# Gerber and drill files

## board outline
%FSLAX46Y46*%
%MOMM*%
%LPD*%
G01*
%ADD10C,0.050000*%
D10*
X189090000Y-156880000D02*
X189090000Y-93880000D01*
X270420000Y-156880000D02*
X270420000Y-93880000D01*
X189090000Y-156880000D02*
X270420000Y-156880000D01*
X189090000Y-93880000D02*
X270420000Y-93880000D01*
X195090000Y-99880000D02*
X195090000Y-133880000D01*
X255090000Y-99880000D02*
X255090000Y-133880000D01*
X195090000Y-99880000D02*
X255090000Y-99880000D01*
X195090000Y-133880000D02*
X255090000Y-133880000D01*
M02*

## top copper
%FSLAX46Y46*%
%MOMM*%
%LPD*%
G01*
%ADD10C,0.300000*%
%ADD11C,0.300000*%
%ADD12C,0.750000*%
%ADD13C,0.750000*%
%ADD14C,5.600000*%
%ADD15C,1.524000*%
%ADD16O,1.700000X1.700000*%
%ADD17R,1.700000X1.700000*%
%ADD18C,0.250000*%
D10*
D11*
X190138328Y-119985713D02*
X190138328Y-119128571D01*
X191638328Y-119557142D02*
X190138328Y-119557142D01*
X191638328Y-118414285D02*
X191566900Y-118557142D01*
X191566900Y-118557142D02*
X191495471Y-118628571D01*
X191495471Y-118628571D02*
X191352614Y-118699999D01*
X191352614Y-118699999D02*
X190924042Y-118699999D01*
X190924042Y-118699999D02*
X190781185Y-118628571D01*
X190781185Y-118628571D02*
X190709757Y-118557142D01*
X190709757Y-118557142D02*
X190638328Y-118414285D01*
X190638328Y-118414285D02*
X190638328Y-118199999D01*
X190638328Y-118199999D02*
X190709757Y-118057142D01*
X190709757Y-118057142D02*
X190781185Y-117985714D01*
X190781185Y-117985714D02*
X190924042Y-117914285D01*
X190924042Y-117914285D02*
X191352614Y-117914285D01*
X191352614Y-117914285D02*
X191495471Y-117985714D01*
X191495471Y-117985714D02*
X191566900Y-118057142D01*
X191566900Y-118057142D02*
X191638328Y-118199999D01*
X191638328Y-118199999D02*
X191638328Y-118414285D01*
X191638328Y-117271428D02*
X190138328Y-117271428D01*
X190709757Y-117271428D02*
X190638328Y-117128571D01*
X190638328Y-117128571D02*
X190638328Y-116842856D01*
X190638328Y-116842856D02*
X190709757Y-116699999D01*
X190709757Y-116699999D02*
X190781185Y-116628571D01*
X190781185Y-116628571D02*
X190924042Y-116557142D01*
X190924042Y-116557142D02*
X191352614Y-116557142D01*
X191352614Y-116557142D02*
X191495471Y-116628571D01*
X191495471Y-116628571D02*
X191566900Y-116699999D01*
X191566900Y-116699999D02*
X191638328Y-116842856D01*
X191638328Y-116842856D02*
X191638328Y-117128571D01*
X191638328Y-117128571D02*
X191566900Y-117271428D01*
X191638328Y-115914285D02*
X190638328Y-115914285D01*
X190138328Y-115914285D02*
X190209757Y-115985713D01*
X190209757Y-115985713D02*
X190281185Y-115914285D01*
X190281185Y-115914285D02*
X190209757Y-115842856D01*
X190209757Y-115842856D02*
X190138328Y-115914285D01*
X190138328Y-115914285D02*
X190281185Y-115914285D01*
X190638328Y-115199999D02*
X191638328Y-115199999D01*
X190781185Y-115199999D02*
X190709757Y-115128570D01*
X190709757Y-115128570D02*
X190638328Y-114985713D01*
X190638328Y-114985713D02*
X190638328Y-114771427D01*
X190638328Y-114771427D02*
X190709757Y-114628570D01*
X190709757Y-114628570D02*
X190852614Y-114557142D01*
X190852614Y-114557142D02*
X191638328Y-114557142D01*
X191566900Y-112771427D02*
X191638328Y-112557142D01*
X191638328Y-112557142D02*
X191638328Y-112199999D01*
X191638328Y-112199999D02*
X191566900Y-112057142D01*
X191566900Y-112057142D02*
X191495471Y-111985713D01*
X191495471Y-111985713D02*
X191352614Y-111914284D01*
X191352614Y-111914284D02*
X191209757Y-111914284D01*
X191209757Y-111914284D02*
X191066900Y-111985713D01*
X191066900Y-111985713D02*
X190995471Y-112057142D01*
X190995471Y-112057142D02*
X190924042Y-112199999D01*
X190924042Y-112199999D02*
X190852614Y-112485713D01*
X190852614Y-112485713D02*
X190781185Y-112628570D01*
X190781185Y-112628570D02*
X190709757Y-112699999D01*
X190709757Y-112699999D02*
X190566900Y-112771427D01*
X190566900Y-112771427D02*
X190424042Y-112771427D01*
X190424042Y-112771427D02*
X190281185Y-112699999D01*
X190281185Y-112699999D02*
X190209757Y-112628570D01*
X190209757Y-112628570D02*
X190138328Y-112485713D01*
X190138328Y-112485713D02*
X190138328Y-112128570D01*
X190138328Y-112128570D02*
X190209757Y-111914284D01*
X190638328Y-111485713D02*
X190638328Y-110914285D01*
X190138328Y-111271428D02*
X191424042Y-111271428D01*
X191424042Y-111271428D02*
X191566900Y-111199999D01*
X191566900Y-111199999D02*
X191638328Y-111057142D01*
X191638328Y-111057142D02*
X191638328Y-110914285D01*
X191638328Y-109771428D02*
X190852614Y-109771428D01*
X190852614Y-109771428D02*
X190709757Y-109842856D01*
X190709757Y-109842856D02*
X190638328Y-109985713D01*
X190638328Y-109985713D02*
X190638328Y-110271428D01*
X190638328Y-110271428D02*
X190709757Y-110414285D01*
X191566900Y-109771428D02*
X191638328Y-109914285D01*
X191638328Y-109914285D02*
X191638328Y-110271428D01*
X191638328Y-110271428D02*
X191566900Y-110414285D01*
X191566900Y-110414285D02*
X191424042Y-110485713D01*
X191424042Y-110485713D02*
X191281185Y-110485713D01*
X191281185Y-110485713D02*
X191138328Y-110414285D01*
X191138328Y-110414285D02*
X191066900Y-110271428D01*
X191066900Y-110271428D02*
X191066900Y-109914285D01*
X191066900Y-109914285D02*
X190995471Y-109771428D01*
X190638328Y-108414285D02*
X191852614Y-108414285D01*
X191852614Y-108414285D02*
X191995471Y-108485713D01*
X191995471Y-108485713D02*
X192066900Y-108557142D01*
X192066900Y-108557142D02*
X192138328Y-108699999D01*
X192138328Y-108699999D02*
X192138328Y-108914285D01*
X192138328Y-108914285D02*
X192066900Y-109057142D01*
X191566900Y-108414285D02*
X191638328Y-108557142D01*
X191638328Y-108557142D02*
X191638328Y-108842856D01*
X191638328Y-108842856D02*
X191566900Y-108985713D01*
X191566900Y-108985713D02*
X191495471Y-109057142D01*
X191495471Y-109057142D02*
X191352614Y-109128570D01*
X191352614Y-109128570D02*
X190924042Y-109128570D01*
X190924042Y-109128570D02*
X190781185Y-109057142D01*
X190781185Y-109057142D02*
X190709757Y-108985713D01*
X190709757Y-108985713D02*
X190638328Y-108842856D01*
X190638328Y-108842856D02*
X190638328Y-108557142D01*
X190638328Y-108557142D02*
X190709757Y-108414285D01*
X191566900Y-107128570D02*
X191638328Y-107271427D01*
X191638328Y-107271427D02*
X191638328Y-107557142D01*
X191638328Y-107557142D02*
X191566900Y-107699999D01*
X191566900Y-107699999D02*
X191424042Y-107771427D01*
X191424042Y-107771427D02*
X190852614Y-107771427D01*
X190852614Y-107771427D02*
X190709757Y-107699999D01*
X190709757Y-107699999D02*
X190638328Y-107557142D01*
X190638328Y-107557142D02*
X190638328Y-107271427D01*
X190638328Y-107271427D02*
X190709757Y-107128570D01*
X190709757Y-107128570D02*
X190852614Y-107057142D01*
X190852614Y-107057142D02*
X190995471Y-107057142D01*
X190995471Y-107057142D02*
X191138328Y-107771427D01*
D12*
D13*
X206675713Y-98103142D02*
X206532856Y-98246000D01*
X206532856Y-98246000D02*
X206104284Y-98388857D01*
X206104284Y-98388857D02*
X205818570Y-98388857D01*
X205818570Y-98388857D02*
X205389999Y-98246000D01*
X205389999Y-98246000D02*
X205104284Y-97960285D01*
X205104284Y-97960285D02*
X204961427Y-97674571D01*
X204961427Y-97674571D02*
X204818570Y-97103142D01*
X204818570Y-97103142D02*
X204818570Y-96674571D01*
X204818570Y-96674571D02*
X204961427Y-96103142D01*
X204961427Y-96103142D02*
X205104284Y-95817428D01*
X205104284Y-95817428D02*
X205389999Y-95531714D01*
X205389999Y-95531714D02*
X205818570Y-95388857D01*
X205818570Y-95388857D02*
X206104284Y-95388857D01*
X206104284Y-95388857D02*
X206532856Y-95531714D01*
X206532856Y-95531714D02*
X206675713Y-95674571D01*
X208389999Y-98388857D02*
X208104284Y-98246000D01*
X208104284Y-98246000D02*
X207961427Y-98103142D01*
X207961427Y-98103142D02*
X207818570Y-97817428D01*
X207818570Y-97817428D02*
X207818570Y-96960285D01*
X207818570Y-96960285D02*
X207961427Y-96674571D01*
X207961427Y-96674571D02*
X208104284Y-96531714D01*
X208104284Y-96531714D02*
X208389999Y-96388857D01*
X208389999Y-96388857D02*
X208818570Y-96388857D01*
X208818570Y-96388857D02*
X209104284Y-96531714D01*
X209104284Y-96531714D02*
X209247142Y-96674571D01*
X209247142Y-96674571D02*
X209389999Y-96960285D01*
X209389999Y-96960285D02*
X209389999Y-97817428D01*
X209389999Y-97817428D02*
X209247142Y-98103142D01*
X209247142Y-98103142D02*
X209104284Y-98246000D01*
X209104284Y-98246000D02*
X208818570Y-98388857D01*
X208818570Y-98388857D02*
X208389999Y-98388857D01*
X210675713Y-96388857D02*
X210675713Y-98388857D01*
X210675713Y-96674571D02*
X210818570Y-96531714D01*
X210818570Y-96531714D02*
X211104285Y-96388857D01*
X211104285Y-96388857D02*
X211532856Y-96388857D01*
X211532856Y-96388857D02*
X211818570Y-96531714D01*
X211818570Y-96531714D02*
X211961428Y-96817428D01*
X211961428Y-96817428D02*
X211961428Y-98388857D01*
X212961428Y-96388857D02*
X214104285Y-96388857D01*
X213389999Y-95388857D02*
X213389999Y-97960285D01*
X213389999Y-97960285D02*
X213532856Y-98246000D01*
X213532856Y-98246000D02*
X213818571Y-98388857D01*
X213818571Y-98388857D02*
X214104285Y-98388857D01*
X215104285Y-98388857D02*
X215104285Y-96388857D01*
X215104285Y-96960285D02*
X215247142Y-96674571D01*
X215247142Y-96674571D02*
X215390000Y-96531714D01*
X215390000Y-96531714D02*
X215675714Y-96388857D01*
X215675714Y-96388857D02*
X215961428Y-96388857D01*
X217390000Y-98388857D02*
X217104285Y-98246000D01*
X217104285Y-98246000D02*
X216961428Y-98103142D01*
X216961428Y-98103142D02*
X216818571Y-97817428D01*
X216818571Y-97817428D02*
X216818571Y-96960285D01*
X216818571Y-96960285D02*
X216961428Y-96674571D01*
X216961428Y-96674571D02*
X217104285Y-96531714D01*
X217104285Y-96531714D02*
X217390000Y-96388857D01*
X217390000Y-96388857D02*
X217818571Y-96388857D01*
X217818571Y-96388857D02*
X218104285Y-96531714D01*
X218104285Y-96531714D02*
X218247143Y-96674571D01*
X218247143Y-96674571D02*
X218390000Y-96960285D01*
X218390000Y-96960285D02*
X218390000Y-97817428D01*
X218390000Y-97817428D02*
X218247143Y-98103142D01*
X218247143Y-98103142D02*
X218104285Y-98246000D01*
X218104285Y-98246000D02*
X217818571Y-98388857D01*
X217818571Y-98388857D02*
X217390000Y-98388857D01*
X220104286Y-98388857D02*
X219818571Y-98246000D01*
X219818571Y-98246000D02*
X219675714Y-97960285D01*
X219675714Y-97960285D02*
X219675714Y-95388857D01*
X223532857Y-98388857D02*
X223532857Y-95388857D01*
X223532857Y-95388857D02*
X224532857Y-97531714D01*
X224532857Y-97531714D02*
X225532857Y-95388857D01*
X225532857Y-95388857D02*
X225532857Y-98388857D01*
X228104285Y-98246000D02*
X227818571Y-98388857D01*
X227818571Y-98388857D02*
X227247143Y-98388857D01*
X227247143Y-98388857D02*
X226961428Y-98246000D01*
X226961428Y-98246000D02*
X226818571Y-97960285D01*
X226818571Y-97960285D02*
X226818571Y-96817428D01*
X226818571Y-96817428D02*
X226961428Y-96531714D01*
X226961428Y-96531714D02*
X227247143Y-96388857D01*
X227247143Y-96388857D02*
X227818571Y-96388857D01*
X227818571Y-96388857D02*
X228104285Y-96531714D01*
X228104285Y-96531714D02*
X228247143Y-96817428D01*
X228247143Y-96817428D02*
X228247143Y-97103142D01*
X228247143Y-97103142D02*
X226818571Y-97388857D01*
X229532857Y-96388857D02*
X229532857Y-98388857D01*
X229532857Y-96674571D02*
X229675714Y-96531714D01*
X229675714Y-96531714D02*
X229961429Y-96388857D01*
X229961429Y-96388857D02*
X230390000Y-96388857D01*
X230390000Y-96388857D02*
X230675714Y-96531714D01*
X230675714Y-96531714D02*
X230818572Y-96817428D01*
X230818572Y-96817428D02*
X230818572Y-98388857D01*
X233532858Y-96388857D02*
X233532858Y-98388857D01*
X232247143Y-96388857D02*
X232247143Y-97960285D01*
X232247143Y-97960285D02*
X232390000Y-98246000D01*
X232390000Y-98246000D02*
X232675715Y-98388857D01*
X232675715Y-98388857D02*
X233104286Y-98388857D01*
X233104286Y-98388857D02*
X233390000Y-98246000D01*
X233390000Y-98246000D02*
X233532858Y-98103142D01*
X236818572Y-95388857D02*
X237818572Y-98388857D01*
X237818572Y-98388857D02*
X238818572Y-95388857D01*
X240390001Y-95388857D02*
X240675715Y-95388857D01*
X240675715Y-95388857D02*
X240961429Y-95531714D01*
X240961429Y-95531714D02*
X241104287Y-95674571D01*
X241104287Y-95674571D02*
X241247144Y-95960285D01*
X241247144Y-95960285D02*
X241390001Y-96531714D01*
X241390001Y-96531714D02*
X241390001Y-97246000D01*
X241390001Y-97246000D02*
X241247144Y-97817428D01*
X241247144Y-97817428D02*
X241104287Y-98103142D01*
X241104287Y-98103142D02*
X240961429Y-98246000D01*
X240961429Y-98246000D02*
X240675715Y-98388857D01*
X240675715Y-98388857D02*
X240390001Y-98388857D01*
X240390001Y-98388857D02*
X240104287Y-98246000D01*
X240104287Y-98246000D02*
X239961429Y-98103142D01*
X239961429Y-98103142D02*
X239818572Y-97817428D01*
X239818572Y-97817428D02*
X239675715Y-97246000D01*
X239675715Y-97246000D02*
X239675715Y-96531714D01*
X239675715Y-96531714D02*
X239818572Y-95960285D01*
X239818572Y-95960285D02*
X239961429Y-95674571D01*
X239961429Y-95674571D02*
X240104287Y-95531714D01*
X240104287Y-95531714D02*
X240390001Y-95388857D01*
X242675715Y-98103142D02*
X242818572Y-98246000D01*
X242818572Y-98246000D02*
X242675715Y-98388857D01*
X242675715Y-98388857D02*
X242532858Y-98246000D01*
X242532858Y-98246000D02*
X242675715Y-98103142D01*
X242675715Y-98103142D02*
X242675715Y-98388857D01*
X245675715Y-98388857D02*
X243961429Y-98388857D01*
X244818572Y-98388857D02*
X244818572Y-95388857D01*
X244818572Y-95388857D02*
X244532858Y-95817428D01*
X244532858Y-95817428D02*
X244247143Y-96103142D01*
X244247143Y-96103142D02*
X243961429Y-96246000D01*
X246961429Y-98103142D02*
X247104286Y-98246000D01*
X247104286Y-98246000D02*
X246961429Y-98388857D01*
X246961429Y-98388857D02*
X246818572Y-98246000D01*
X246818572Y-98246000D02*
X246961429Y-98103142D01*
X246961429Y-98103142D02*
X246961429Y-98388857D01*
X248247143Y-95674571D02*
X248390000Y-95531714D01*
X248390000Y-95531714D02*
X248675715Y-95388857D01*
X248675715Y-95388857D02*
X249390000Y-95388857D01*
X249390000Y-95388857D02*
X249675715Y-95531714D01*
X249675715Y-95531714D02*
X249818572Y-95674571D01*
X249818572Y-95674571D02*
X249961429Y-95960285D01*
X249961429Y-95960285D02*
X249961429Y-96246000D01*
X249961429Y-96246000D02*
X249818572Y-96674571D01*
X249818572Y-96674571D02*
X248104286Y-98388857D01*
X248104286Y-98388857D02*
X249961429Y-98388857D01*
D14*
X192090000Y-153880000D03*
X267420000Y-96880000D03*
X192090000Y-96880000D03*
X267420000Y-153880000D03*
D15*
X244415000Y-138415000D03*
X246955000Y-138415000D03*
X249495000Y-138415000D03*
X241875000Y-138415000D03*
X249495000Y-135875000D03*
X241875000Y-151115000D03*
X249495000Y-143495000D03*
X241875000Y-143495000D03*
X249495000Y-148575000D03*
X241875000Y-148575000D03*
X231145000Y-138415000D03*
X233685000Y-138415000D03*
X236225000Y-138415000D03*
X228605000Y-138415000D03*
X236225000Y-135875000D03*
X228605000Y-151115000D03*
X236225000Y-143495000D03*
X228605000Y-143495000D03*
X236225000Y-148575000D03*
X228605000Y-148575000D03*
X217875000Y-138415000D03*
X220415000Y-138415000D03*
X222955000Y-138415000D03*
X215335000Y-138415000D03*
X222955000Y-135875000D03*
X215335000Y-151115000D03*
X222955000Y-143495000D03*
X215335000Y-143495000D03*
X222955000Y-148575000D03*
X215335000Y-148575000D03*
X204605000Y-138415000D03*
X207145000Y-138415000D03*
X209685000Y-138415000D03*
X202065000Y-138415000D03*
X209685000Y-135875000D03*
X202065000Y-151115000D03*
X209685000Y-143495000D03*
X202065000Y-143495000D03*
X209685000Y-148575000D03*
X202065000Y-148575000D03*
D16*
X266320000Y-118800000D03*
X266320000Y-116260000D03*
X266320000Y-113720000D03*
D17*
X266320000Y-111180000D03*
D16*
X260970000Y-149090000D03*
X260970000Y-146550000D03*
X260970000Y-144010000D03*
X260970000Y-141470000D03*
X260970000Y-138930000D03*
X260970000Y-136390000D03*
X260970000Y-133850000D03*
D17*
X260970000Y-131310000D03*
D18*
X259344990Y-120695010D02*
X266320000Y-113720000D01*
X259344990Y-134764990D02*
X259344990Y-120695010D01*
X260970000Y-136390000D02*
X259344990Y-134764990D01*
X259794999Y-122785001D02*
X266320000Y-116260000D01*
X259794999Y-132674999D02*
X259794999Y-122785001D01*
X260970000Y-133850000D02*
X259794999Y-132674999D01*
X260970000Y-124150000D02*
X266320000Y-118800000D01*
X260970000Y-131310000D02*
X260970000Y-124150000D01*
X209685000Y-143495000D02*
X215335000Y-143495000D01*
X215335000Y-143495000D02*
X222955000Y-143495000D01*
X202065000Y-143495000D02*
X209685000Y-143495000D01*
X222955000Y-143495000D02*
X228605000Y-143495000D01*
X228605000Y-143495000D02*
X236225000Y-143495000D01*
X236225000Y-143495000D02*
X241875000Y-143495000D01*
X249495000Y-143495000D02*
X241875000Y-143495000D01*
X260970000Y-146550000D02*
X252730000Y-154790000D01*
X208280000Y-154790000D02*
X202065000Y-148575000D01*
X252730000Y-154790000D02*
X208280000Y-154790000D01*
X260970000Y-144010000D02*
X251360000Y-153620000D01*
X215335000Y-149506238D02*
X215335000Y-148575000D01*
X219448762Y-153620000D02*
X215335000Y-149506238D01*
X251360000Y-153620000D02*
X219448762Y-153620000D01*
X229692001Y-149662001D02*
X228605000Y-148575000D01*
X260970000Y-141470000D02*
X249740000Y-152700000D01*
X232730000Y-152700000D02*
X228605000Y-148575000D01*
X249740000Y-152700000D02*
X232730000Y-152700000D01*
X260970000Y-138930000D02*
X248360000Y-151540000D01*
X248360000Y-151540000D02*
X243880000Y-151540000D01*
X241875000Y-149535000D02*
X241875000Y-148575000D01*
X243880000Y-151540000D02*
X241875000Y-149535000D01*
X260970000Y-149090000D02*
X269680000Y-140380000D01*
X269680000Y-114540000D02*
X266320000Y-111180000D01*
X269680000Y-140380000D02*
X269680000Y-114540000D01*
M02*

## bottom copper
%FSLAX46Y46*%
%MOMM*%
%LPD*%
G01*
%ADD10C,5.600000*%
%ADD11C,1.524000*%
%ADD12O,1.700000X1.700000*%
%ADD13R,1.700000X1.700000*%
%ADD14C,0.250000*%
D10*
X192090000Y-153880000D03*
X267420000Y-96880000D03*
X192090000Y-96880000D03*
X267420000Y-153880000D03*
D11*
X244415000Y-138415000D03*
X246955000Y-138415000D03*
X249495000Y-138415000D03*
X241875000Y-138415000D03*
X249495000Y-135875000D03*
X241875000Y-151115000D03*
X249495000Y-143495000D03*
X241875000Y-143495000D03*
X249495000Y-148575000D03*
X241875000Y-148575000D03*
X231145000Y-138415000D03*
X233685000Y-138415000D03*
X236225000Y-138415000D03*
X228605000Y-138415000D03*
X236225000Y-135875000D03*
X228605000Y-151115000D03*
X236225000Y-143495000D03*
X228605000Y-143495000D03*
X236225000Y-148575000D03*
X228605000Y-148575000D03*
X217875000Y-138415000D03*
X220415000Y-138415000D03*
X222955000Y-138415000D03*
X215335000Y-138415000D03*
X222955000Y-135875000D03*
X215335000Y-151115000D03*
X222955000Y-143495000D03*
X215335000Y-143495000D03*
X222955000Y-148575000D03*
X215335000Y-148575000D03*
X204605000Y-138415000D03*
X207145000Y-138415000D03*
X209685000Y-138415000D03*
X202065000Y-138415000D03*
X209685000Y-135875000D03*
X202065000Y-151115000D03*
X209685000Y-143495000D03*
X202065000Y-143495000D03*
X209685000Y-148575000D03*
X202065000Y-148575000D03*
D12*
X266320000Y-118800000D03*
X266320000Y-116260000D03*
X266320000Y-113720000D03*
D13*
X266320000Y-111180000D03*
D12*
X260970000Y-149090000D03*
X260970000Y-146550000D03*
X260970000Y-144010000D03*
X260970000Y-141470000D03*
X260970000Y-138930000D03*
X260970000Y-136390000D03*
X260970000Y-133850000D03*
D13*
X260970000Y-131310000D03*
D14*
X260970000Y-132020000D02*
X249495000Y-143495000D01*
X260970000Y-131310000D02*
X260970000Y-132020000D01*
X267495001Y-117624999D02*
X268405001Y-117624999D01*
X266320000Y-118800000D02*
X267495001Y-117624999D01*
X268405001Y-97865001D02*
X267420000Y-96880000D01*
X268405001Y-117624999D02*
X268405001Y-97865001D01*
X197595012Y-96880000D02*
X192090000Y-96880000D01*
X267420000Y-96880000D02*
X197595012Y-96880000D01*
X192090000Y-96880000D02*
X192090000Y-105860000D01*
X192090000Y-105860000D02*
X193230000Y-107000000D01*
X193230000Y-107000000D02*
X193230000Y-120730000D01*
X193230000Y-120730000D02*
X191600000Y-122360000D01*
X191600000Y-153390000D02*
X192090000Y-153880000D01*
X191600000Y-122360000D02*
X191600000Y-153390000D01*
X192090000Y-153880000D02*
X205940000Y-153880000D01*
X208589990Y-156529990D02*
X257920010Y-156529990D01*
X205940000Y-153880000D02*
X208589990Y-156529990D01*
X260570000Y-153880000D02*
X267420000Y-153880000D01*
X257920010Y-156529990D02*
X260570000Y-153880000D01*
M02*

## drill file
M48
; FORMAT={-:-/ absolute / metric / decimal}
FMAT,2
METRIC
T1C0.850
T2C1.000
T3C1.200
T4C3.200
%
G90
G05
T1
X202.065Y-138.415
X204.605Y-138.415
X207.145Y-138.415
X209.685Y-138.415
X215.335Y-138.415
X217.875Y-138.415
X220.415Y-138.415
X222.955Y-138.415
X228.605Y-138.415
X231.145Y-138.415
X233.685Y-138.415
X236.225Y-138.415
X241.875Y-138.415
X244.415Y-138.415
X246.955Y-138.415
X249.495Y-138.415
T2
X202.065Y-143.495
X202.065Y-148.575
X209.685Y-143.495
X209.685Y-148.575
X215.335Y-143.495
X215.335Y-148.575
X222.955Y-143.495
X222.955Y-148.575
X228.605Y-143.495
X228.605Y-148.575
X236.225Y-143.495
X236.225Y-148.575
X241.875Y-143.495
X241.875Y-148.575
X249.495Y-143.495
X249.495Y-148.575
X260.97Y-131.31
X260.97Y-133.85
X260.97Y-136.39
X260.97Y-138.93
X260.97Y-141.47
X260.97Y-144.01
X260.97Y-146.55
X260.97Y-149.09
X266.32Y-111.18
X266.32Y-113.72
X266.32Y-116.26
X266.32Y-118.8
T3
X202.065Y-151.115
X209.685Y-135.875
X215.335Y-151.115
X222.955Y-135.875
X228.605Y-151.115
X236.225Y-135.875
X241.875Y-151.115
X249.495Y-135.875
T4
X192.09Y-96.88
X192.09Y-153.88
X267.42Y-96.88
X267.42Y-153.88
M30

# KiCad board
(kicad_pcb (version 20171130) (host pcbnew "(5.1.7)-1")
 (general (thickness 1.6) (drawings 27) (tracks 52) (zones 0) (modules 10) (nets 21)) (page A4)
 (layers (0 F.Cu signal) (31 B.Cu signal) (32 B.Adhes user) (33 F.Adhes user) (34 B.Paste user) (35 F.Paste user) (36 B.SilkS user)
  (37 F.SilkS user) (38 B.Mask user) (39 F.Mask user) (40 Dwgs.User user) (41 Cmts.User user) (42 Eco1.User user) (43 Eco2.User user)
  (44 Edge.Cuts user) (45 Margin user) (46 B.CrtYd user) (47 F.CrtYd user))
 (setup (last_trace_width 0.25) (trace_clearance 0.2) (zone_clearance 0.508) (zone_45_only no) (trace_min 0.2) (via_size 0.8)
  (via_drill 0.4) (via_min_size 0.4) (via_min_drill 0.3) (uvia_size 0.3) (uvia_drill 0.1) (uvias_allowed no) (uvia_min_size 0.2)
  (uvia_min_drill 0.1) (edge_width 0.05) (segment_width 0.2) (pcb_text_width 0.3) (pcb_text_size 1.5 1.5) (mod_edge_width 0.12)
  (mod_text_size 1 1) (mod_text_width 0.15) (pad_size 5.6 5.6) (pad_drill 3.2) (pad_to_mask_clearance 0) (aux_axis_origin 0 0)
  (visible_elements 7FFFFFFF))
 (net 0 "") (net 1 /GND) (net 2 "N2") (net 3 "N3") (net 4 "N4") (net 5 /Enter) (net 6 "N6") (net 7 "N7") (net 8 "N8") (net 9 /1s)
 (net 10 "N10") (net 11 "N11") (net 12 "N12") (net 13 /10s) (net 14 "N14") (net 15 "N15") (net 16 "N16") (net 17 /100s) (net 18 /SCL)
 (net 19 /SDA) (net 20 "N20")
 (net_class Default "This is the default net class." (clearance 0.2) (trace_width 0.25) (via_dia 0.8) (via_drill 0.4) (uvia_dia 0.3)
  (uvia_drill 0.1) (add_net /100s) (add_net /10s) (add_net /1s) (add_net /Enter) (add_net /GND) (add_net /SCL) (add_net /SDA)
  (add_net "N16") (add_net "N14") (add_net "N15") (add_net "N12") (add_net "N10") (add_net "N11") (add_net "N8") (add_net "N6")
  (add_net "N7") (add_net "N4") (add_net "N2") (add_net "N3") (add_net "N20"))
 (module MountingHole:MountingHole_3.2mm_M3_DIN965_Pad (layer F.Cu) (at 192.09 153.88)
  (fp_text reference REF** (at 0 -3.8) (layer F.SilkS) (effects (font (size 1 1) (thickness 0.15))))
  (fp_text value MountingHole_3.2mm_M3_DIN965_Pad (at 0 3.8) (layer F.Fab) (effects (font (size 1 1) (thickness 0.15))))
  (pad 1 thru_hole circle (at 0 0) (size 5.6 5.6) (drill 3.2) (layers *.Cu *.Mask) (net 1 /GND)))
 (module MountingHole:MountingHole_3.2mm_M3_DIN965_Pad (layer F.Cu) (at 267.42 96.88)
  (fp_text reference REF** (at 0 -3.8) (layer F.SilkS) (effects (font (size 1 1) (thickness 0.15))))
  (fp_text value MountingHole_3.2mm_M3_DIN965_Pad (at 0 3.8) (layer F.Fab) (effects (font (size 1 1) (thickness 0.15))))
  (pad 1 thru_hole circle (at 0 0) (size 5.6 5.6) (drill 3.2) (layers *.Cu *.Mask) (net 1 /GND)))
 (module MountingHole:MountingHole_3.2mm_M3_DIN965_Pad (layer F.Cu) (at 192.09 96.88)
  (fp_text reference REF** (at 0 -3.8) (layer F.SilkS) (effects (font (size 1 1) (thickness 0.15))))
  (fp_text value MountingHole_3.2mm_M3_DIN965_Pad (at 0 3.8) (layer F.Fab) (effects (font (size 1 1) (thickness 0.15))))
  (pad 1 thru_hole circle (at 0 0) (size 5.6 5.6) (drill 3.2) (layers *.Cu *.Mask) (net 1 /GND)))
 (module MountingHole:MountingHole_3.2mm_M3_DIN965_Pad (layer F.Cu) (at 267.42 153.88)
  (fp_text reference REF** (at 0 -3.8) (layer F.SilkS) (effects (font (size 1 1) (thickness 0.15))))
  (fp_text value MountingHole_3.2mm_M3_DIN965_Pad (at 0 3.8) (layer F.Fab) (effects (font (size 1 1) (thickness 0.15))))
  (pad 1 thru_hole circle (at 0 0) (size 5.6 5.6) (drill 3.2) (layers *.Cu *.Mask) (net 1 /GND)))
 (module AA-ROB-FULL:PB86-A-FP (layer F.Cu) (at 239.515 134.995)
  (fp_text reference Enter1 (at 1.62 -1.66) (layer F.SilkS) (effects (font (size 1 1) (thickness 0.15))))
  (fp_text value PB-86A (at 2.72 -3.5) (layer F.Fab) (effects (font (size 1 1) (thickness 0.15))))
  (pad 5 thru_hole circle (at 4.9 3.42) (size 1.524 1.524) (drill 0.85) (layers *.Cu *.Mask) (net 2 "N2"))
  (pad 6 thru_hole circle (at 7.44 3.42) (size 1.524 1.524) (drill 0.85) (layers *.Cu *.Mask) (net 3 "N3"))
  (pad 7 thru_hole circle (at 9.98 3.42) (size 1.524 1.524) (drill 0.85) (layers *.Cu *.Mask))
  (pad 4 thru_hole circle (at 2.36 3.42) (size 1.524 1.524) (drill 0.85) (layers *.Cu *.Mask))
  (pad 8 thru_hole circle (at 9.98 0.88) (size 1.524 1.524) (drill 1.2) (layers *.Cu *.Mask))
  (pad 8 thru_hole circle (at 2.36 16.12) (size 1.524 1.524) (drill 1.2) (layers *.Cu *.Mask))
  (pad 1 thru_hole circle (at 9.98 8.5) (size 1.524 1.524) (drill 1) (layers *.Cu *.Mask) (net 1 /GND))
  (pad 1 thru_hole circle (at 2.36 8.5) (size 1.524 1.524) (drill 1) (layers *.Cu *.Mask) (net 1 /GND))
  (pad 3 thru_hole circle (at 9.98 13.58) (size 1.524 1.524) (drill 1) (layers *.Cu *.Mask) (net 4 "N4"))
  (pad 2 thru_hole circle (at 2.36 13.58) (size 1.524 1.524) (drill 1) (layers *.Cu *.Mask) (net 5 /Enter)))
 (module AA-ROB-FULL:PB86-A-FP (layer F.Cu) (at 226.245 134.995)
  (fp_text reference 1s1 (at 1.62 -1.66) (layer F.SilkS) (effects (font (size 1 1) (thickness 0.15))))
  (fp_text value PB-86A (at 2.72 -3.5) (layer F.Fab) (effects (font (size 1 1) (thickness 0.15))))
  (pad 5 thru_hole circle (at 4.9 3.42) (size 1.524 1.524) (drill 0.85) (layers *.Cu *.Mask) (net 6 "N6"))
  (pad 6 thru_hole circle (at 7.44 3.42) (size 1.524 1.524) (drill 0.85) (layers *.Cu *.Mask) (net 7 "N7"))
  (pad 7 thru_hole circle (at 9.98 3.42) (size 1.524 1.524) (drill 0.85) (layers *.Cu *.Mask))
  (pad 4 thru_hole circle (at 2.36 3.42) (size 1.524 1.524) (drill 0.85) (layers *.Cu *.Mask))
  (pad 8 thru_hole circle (at 9.98 0.88) (size 1.524 1.524) (drill 1.2) (layers *.Cu *.Mask))
  (pad 8 thru_hole circle (at 2.36 16.12) (size 1.524 1.524) (drill 1.2) (layers *.Cu *.Mask))
  (pad 1 thru_hole circle (at 9.98 8.5) (size 1.524 1.524) (drill 1) (layers *.Cu *.Mask) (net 1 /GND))
  (pad 1 thru_hole circle (at 2.36 8.5) (size 1.524 1.524) (drill 1) (layers *.Cu *.Mask) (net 1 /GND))
  (pad 3 thru_hole circle (at 9.98 13.58) (size 1.524 1.524) (drill 1) (layers *.Cu *.Mask) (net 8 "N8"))
  (pad 2 thru_hole circle (at 2.36 13.58) (size 1.524 1.524) (drill 1) (layers *.Cu *.Mask) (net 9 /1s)))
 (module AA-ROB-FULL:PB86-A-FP (layer F.Cu) (at 212.975 134.995)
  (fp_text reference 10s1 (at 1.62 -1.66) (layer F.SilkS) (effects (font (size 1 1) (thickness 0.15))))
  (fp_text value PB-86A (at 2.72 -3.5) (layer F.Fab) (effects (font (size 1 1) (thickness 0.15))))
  (pad 5 thru_hole circle (at 4.9 3.42) (size 1.524 1.524) (drill 0.85) (layers *.Cu *.Mask) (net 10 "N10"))
  (pad 6 thru_hole circle (at 7.44 3.42) (size 1.524 1.524) (drill 0.85) (layers *.Cu *.Mask) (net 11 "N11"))
  (pad 7 thru_hole circle (at 9.98 3.42) (size 1.524 1.524) (drill 0.85) (layers *.Cu *.Mask))
  (pad 4 thru_hole circle (at 2.36 3.42) (size 1.524 1.524) (drill 0.85) (layers *.Cu *.Mask))
  (pad 8 thru_hole circle (at 9.98 0.88) (size 1.524 1.524) (drill 1.2) (layers *.Cu *.Mask))
  (pad 8 thru_hole circle (at 2.36 16.12) (size 1.524 1.524) (drill 1.2) (layers *.Cu *.Mask))
  (pad 1 thru_hole circle (at 9.98 8.5) (size 1.524 1.524) (drill 1) (layers *.Cu *.Mask) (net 1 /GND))
  (pad 1 thru_hole circle (at 2.36 8.5) (size 1.524 1.524) (drill 1) (layers *.Cu *.Mask) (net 1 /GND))
  (pad 3 thru_hole circle (at 9.98 13.58) (size 1.524 1.524) (drill 1) (layers *.Cu *.Mask) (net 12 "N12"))
  (pad 2 thru_hole circle (at 2.36 13.58) (size 1.524 1.524) (drill 1) (layers *.Cu *.Mask) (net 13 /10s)))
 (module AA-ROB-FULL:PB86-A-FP (layer F.Cu) (at 199.705 134.995)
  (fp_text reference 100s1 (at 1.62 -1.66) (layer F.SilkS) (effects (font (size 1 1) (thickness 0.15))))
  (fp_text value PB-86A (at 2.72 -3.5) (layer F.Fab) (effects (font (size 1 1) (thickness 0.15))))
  (pad 5 thru_hole circle (at 4.9 3.42) (size 1.524 1.524) (drill 0.85) (layers *.Cu *.Mask) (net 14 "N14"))
  (pad 6 thru_hole circle (at 7.44 3.42) (size 1.524 1.524) (drill 0.85) (layers *.Cu *.Mask) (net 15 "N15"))
  (pad 7 thru_hole circle (at 9.98 3.42) (size 1.524 1.524) (drill 0.85) (layers *.Cu *.Mask))
  (pad 4 thru_hole circle (at 2.36 3.42) (size 1.524 1.524) (drill 0.85) (layers *.Cu *.Mask))
  (pad 8 thru_hole circle (at 9.98 0.88) (size 1.524 1.524) (drill 1.2) (layers *.Cu *.Mask))
  (pad 8 thru_hole circle (at 2.36 16.12) (size 1.524 1.524) (drill 1.2) (layers *.Cu *.Mask))
  (pad 1 thru_hole circle (at 9.98 8.5) (size 1.524 1.524) (drill 1) (layers *.Cu *.Mask) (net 1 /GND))
  (pad 1 thru_hole circle (at 2.36 8.5) (size 1.524 1.524) (drill 1) (layers *.Cu *.Mask) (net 1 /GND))
  (pad 3 thru_hole circle (at 9.98 13.58) (size 1.524 1.524) (drill 1) (layers *.Cu *.Mask) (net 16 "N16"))
  (pad 2 thru_hole circle (at 2.36 13.58) (size 1.524 1.524) (drill 1) (layers *.Cu *.Mask) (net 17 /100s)))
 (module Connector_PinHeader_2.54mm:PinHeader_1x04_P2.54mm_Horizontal (layer B.Cu) (at 266.32 111.18 180)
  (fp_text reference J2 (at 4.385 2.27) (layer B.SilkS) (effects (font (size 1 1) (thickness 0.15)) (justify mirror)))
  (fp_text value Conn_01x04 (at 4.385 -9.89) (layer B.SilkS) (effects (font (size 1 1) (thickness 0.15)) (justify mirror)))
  (pad 4 thru_hole oval (at 0 -7.62 180) (size 1.7 1.7) (drill 1) (layers *.Cu *.Mask) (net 1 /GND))
  (pad 3 thru_hole oval (at 0 -5.08 180) (size 1.7 1.7) (drill 1) (layers *.Cu *.Mask) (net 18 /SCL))
  (pad 2 thru_hole oval (at 0 -2.54 180) (size 1.7 1.7) (drill 1) (layers *.Cu *.Mask) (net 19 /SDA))
  (pad 1 thru_hole rect (at 0 0 180) (size 1.7 1.7) (drill 1) (layers *.Cu *.Mask) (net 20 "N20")))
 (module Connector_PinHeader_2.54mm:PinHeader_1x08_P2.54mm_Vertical (layer F.Cu) (at 260.97 131.31)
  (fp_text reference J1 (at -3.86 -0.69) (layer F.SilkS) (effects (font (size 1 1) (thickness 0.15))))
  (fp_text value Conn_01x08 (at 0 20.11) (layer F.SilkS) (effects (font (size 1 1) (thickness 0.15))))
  (pad 8 thru_hole oval (at 0 17.78) (size 1.7 1.7) (drill 1) (layers *.Cu *.Mask) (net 20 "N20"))
  (pad 7 thru_hole oval (at 0 15.24) (size 1.7 1.7) (drill 1) (layers *.Cu *.Mask) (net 17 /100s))
  (pad 6 thru_hole oval (at 0 12.7) (size 1.7 1.7) (drill 1) (layers *.Cu *.Mask) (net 13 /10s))
  (pad 5 thru_hole oval (at 0 10.16) (size 1.7 1.7) (drill 1) (layers *.Cu *.Mask) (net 9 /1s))
  (pad 4 thru_hole oval (at 0 7.62) (size 1.7 1.7) (drill 1) (layers *.Cu *.Mask) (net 5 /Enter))
  (pad 3 thru_hole oval (at 0 5.08) (size 1.7 1.7) (drill 1) (layers *.Cu *.Mask) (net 19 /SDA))
  (pad 2 thru_hole oval (at 0 2.54) (size 1.7 1.7) (drill 1) (layers *.Cu *.Mask) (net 18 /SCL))
  (pad 1 thru_hole rect (at 0 0) (size 1.7 1.7) (drill 1) (layers *.Cu *.Mask) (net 1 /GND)))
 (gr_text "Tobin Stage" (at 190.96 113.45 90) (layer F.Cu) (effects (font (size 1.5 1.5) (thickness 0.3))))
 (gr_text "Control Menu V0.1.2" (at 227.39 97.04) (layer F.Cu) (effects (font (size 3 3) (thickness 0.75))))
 (gr_line (start 189.09 156.88) (end 189.09 93.88) (layer Edge.Cuts) (width 0.05))
 (gr_line (start 270.42 156.88) (end 270.42 93.88) (layer Edge.Cuts) (width 0.05))
 (gr_line (start 189.09 156.88) (end 270.42 156.88) (layer Edge.Cuts) (width 0.05))
 (gr_line (start 189.09 93.88) (end 270.42 93.88) (layer Edge.Cuts) (width 0.05))
 (gr_line (start 195.09 99.88) (end 195.09 133.88) (layer Edge.Cuts) (width 0.05))
 (gr_line (start 255.09 99.88) (end 255.09 133.88) (layer Edge.Cuts) (width 0.05))
 (gr_line (start 195.09 99.88) (end 255.09 99.88) (layer Edge.Cuts) (width 0.05))
 (gr_line (start 195.09 133.88) (end 255.09 133.88) (layer Edge.Cuts) (width 0.05))
 (segment (start 259.34499 120.69501) (end 266.32 113.72) (width 0.25) (layer F.Cu) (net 19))
 (segment (start 259.34499 134.76499) (end 259.34499 120.69501) (width 0.25) (layer F.Cu) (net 19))
 (segment (start 260.97 136.39) (end 259.34499 134.76499) (width 0.25) (layer F.Cu) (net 19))
 (segment (start 259.794999 122.785001) (end 266.32 116.26) (width 0.25) (layer F.Cu) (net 18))
 (segment (start 259.794999 132.674999) (end 259.794999 122.785001) (width 0.25) (layer F.Cu) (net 18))
 (segment (start 260.97 133.85) (end 259.794999 132.674999) (width 0.25) (layer F.Cu) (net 18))
 (segment (start 260.97 124.15) (end 266.32 118.8) (width 0.25) (layer F.Cu) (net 1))
 (segment (start 260.97 131.31) (end 260.97 124.15) (width 0.25) (layer F.Cu) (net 1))
 (segment (start 209.685 143.495) (end 215.335 143.495) (width 0.25) (layer F.Cu) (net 1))
 (segment (start 215.335 143.495) (end 222.955 143.495) (width 0.25) (layer F.Cu) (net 1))
 (segment (start 202.065 143.495) (end 209.685 143.495) (width 0.25) (layer F.Cu) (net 1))
 (segment (start 222.955 143.495) (end 228.605 143.495) (width 0.25) (layer F.Cu) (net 1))
 (segment (start 228.605 143.495) (end 236.225 143.495) (width 0.25) (layer F.Cu) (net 1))
 (segment (start 236.225 143.495) (end 241.875 143.495) (width 0.25) (layer F.Cu) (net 1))
 (segment (start 249.495 143.495) (end 241.875 143.495) (width 0.25) (layer F.Cu) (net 1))
 (segment (start 260.97 132.02) (end 249.495 143.495) (width 0.25) (layer B.Cu) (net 1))
 (segment (start 260.97 131.31) (end 260.97 132.02) (width 0.25) (layer B.Cu) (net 1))
 (segment (start 267.495001 117.624999) (end 268.405001 117.624999) (width 0.25) (layer B.Cu) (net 1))
 (segment (start 266.32 118.8) (end 267.495001 117.624999) (width 0.25) (layer B.Cu) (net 1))
 (segment (start 268.405001 97.865001) (end 267.42 96.88) (width 0.25) (layer B.Cu) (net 1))
 (segment (start 268.405001 117.624999) (end 268.405001 97.865001) (width 0.25) (layer B.Cu) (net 1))
 (segment (start 197.595012 96.88) (end 192.09 96.88) (width 0.25) (layer B.Cu) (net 1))
 (segment (start 267.42 96.88) (end 197.595012 96.88) (width 0.25) (layer B.Cu) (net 1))
 (segment (start 192.09 96.88) (end 192.09 105.86) (width 0.25) (layer B.Cu) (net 1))
 (segment (start 192.09 105.86) (end 193.23 107) (width 0.25) (layer B.Cu) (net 1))
 (segment (start 193.23 107) (end 193.23 120.73) (width 0.25) (layer B.Cu) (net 1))
 (segment (start 193.23 120.73) (end 191.6 122.36) (width 0.25) (layer B.Cu) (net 1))
 (segment (start 191.6 153.39) (end 192.09 153.88) (width 0.25) (layer B.Cu) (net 1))
 (segment (start 191.6 122.36) (end 191.6 153.39) (width 0.25) (layer B.Cu) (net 1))
 (segment (start 192.09 153.88) (end 205.94 153.88) (width 0.25) (layer B.Cu) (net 1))
 (segment (start 208.58999 156.52999) (end 257.92001 156.52999) (width 0.25) (layer B.Cu) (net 1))
 (segment (start 205.94 153.88) (end 208.58999 156.52999) (width 0.25) (layer B.Cu) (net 1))
 (segment (start 260.57 153.88) (end 267.42 153.88) (width 0.25) (layer B.Cu) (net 1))
 (segment (start 257.92001 156.52999) (end 260.57 153.88) (width 0.25) (layer B.Cu) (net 1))
 (segment (start 260.97 146.55) (end 252.73 154.79) (width 0.25) (layer F.Cu) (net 17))
 (segment (start 208.28 154.79) (end 202.065 148.575) (width 0.25) (layer F.Cu) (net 17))
 (segment (start 252.73 154.79) (end 208.28 154.79) (width 0.25) (layer F.Cu) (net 17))
 (segment (start 260.97 144.01) (end 251.36 153.62) (width 0.25) (layer F.Cu) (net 13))
 (segment (start 215.335 149.506238) (end 215.335 148.575) (width 0.25) (layer F.Cu) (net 13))
 (segment (start 219.448762 153.62) (end 215.335 149.506238) (width 0.25) (layer F.Cu) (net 13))
 (segment (start 251.36 153.62) (end 219.448762 153.62) (width 0.25) (layer F.Cu) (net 13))
 (segment (start 229.692001 149.662001) (end 228.605 148.575) (width 0.25) (layer F.Cu) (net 9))
 (segment (start 260.97 141.47) (end 249.74 152.7) (width 0.25) (layer F.Cu) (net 9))
 (segment (start 232.73 152.7) (end 228.605 148.575) (width 0.25) (layer F.Cu) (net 9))
 (segment (start 249.74 152.7) (end 232.73 152.7) (width 0.25) (layer F.Cu) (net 9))
 (segment (start 260.97 138.93) (end 248.36 151.54) (width 0.25) (layer F.Cu) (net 5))
 (segment (start 248.36 151.54) (end 243.88 151.54) (width 0.25) (layer F.Cu) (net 5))
 (segment (start 241.875 149.535) (end 241.875 148.575) (width 0.25) (layer F.Cu) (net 5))
 (segment (start 243.88 151.54) (end 241.875 149.535) (width 0.25) (layer F.Cu) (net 5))
 (segment (start 260.97 149.09) (end 269.68 140.38) (width 0.25) (layer F.Cu) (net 20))
 (segment (start 269.68 114.54) (end 266.32 111.18) (width 0.25) (layer F.Cu) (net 20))
 (segment (start 269.68 140.38) (end 269.68 114.54) (width 0.25) (layer F.Cu) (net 20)))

